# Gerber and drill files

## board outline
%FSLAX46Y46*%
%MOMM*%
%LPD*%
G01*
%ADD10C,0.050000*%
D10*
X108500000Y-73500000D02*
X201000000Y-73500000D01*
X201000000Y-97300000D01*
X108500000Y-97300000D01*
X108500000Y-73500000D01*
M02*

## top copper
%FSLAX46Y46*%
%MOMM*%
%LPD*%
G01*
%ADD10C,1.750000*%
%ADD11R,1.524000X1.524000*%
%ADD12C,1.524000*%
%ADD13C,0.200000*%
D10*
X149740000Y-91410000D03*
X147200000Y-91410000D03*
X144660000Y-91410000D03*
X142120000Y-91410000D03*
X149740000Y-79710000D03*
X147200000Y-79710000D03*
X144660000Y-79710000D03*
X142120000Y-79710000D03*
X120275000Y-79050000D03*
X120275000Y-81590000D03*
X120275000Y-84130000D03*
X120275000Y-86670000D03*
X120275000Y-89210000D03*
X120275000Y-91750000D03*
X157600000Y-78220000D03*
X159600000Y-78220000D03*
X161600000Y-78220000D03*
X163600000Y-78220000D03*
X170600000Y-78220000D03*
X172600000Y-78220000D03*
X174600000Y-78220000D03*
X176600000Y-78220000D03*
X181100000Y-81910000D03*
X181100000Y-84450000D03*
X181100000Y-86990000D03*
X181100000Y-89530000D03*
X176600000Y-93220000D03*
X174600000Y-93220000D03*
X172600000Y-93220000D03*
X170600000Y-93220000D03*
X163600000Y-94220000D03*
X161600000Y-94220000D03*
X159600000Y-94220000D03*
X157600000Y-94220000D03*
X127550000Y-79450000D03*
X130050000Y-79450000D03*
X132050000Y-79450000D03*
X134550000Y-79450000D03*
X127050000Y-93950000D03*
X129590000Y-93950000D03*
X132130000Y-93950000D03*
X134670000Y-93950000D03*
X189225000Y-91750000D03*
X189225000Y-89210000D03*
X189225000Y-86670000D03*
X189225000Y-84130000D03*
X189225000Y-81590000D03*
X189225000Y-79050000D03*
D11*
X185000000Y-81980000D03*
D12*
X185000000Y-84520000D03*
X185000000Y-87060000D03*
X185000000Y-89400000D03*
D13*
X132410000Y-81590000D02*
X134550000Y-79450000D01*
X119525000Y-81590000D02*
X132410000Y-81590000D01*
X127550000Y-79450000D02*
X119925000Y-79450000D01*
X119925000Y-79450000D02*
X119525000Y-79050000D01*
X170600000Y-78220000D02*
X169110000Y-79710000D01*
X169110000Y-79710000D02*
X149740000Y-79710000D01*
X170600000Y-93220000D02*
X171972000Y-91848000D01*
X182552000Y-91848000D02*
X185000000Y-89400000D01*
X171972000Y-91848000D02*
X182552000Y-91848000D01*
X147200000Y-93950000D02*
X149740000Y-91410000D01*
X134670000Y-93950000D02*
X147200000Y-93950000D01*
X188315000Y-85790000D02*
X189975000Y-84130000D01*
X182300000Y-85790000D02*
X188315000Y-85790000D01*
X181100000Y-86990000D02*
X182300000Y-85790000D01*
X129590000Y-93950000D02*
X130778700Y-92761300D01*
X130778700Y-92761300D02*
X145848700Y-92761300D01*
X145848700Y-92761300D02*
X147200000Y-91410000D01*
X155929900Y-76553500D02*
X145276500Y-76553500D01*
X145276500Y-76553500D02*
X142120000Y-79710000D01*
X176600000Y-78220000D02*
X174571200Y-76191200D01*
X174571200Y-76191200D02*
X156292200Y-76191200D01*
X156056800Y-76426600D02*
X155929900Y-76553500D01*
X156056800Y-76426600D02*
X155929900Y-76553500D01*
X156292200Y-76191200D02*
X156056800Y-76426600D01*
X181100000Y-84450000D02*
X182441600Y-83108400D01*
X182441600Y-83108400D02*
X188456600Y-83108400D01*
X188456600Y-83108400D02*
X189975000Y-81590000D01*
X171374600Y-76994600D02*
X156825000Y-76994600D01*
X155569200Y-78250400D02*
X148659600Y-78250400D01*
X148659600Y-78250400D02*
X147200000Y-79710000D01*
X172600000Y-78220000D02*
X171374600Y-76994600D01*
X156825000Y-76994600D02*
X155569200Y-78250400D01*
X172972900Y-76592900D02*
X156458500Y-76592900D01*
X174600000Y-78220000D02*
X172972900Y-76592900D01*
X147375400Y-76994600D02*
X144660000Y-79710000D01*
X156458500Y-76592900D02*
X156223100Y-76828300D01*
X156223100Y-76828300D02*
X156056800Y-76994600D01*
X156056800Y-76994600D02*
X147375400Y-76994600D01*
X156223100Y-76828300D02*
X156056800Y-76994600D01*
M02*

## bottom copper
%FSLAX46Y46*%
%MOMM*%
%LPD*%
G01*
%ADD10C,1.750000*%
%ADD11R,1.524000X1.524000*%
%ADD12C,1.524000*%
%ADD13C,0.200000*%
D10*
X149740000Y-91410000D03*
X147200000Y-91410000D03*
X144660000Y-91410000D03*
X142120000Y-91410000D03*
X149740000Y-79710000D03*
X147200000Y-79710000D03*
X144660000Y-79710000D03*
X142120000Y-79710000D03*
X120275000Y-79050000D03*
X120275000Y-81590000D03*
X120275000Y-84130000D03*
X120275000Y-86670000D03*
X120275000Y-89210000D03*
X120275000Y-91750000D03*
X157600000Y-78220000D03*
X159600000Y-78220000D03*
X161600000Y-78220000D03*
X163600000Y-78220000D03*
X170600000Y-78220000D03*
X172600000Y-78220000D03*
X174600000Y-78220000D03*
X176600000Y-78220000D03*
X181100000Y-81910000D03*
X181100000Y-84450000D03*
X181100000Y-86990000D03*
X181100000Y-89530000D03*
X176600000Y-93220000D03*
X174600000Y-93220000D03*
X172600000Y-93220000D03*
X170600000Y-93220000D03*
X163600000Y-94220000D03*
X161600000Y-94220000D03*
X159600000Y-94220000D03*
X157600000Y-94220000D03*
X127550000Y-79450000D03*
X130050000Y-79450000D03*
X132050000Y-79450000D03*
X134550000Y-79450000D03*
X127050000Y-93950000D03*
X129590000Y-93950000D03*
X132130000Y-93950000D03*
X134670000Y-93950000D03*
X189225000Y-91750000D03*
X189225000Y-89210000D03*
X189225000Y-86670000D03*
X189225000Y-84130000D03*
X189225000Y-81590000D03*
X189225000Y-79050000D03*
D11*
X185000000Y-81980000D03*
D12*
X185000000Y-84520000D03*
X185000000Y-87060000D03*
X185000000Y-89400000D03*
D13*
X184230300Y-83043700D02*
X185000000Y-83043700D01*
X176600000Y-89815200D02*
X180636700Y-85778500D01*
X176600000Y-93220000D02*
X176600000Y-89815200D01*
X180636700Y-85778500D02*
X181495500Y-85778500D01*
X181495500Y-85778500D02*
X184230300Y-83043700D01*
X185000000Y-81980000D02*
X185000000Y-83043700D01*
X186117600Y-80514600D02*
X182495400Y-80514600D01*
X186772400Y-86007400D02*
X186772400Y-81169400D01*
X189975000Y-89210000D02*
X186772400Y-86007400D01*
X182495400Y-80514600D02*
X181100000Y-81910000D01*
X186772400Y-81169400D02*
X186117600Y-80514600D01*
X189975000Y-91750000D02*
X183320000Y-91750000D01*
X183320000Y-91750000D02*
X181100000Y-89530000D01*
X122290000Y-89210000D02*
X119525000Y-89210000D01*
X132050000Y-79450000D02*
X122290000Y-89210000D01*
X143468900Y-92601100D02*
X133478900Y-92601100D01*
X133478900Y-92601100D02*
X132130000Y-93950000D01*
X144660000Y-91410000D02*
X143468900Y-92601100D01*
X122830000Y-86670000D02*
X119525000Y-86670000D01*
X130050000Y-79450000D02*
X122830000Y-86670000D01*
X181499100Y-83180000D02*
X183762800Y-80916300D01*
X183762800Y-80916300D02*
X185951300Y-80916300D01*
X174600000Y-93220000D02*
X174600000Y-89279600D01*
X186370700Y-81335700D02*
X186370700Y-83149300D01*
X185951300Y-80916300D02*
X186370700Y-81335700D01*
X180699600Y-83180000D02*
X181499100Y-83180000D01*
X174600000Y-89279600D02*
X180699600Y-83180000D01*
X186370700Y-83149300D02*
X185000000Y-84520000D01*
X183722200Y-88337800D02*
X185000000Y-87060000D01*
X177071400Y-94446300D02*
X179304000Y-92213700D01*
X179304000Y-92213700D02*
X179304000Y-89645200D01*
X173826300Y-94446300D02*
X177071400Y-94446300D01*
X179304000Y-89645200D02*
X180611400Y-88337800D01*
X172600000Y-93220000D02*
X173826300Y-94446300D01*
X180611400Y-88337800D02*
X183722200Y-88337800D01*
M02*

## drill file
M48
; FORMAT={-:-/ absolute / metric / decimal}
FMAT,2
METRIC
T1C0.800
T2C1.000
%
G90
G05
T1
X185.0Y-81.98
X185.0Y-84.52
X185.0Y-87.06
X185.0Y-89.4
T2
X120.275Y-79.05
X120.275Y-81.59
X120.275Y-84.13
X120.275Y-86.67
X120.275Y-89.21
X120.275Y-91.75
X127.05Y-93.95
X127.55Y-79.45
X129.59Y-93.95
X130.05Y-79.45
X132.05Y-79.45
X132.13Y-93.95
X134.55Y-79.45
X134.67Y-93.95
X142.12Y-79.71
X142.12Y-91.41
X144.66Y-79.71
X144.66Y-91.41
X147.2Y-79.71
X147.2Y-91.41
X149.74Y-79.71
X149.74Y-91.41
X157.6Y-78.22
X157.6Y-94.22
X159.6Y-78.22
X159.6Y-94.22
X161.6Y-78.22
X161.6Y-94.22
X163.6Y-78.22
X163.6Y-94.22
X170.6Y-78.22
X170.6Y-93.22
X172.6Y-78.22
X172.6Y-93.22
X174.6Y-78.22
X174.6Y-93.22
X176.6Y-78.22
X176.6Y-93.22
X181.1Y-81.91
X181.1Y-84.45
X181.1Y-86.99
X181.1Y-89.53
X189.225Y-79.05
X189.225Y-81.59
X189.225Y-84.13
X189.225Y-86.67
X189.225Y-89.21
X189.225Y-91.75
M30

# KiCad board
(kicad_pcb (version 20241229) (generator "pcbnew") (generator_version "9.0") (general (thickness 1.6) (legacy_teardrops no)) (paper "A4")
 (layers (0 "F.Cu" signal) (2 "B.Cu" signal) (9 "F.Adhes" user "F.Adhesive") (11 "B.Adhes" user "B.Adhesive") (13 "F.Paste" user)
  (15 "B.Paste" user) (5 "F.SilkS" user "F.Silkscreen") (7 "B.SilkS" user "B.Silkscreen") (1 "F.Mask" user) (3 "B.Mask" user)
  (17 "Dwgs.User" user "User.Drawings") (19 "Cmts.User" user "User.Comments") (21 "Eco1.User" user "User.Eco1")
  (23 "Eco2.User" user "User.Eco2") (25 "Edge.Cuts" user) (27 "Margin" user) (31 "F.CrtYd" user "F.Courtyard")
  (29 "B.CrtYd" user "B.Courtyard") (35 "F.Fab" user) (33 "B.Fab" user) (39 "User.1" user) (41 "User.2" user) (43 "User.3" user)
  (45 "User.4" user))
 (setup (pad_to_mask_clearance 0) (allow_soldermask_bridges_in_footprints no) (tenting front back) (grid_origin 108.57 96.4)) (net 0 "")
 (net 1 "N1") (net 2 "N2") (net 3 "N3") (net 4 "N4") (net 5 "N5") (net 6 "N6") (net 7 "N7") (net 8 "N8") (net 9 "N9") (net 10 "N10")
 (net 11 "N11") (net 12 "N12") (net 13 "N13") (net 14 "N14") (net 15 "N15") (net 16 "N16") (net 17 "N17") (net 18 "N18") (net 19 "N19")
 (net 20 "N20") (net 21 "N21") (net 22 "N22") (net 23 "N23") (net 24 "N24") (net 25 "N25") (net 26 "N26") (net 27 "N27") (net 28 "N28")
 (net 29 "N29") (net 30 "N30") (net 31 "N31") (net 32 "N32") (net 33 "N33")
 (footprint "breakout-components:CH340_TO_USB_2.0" (layer "F.Cu") (at 151.68 92.91 180)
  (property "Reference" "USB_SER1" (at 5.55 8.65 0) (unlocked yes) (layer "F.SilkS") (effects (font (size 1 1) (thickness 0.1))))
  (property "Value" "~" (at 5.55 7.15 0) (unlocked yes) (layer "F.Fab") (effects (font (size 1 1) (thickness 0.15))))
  (pad "1" thru_hole circle (at 1.94 1.5 180) (size 1.75 1.75) (drill 1) (layers "*.Cu" "*.Mask") (remove_unused_layers no) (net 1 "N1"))
  (pad "2" thru_hole circle (at 4.48 1.5 180) (size 1.75 1.75) (drill 1) (layers "*.Cu" "*.Mask") (remove_unused_layers no) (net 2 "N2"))
  (pad "3" thru_hole circle (at 7.02 1.5 180) (size 1.75 1.75) (drill 1) (layers "*.Cu" "*.Mask") (remove_unused_layers no) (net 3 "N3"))
  (pad "4" thru_hole circle (at 9.56 1.5 180) (size 1.75 1.75) (drill 1) (layers "*.Cu" "*.Mask") (remove_unused_layers no) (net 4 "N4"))
  (pad "5" thru_hole circle (at 1.94 13.2 180) (size 1.75 1.75) (drill 1) (layers "*.Cu" "*.Mask") (remove_unused_layers no) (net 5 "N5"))
  (pad "6" thru_hole circle (at 4.48 13.2 180) (size 1.75 1.75) (drill 1) (layers "*.Cu" "*.Mask") (remove_unused_layers no) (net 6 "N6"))
  (pad "7" thru_hole circle (at 7.02 13.2 180) (size 1.75 1.75) (drill 1) (layers "*.Cu" "*.Mask") (remove_unused_layers no) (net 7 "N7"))
  (pad "8" thru_hole circle (at 9.56 13.2 180) (size 1.75 1.75) (drill 1) (layers "*.Cu" "*.Mask") (remove_unused_layers no) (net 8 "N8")))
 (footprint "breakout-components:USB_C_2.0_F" (layer "F.Cu") (at 108.525 74.5)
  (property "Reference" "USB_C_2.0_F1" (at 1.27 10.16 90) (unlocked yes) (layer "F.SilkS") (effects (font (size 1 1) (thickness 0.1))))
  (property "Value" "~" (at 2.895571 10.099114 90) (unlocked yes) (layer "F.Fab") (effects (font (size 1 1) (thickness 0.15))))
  (pad "1" thru_hole circle (at 11.75 4.55) (size 1.75 1.75) (drill 1) (layers "*.Cu" "*.Mask") (remove_unused_layers no) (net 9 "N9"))
  (pad "2" thru_hole circle (at 11.75 7.09) (size 1.75 1.75) (drill 1) (layers "*.Cu" "*.Mask") (remove_unused_layers no) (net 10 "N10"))
  (pad "3" thru_hole circle (at 11.75 9.63) (size 1.75 1.75) (drill 1) (layers "*.Cu" "*.Mask") (remove_unused_layers no) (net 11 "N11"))
  (pad "4" thru_hole circle (at 11.75 12.17) (size 1.75 1.75) (drill 1) (layers "*.Cu" "*.Mask") (remove_unused_layers no) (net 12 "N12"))
  (pad "5" thru_hole circle (at 11.75 14.71) (size 1.75 1.75) (drill 1) (layers "*.Cu" "*.Mask") (remove_unused_layers no) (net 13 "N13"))
  (pad "6" thru_hole circle (at 11.75 17.25) (size 1.75 1.75) (drill 1) (layers "*.Cu" "*.Mask") (remove_unused_layers no) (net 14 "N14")))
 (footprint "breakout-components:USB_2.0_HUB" (layer "F.Cu") (at 153.6 95.22 90)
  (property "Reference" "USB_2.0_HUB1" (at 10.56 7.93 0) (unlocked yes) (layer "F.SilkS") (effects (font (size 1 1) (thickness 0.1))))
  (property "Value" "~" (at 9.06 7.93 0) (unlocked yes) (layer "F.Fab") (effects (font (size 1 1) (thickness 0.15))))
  (pad "1" thru_hole circle (at 17 4 90) (size 1.75 1.75) (drill 1) (layers "*.Cu" "*.Mask") (remove_unused_layers no) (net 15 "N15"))
  (pad "2" thru_hole circle (at 17 6 90) (size 1.75 1.75) (drill 1) (layers "*.Cu" "*.Mask") (remove_unused_layers no) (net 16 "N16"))
  (pad "3" thru_hole circle (at 17 8 90) (size 1.75 1.75) (drill 1) (layers "*.Cu" "*.Mask") (remove_unused_layers no) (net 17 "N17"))
  (pad "4" thru_hole circle (at 17 10 90) (size 1.75 1.75) (drill 1) (layers "*.Cu" "*.Mask") (remove_unused_layers no) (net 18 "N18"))
  (pad "5" thru_hole circle (at 17 17 90) (size 1.75 1.75) (drill 1) (layers "*.Cu" "*.Mask") (remove_unused_layers no) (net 5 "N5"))
  (pad "6" thru_hole circle (at 17 19 90) (size 1.75 1.75) (drill 1) (layers "*.Cu" "*.Mask") (remove_unused_layers no) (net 6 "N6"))
  (pad "7" thru_hole circle (at 17 21 90) (size 1.75 1.75) (drill 1) (layers "*.Cu" "*.Mask") (remove_unused_layers no) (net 7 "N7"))
  (pad "8" thru_hole circle (at 17 23 90) (size 1.75 1.75) (drill 1) (layers "*.Cu" "*.Mask") (remove_unused_layers no) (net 8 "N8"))
  (pad "9" thru_hole circle (at 13.31 27.5 90) (size 1.75 1.75) (drill 1) (layers "*.Cu" "*.Mask") (remove_unused_layers no) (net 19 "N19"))
  (pad "10" thru_hole circle (at 10.77 27.5 90) (size 1.75 1.75) (drill 1) (layers "*.Cu" "*.Mask") (remove_unused_layers no) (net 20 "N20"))
  (pad "11" thru_hole circle (at 8.23 27.5 90) (size 1.75 1.75) (drill 1) (layers "*.Cu" "*.Mask") (remove_unused_layers no) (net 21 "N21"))
  (pad "12" thru_hole circle (at 5.69 27.5 90) (size 1.75 1.75) (drill 1) (layers "*.Cu" "*.Mask") (remove_unused_layers no) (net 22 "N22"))
  (pad "13" thru_hole circle (at 2 23 90) (size 1.75 1.75) (drill 1) (layers "*.Cu" "*.Mask") (remove_unused_layers no) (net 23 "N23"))
  (pad "14" thru_hole circle (at 2 21 90) (size 1.75 1.75) (drill 1) (layers "*.Cu" "*.Mask") (remove_unused_layers no) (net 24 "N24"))
  (pad "15" thru_hole circle (at 2 19 90) (size 1.75 1.75) (drill 1) (layers "*.Cu" "*.Mask") (remove_unused_layers no) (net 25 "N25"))
  (pad "16" thru_hole circle (at 2 17 90) (size 1.75 1.75) (drill 1) (layers "*.Cu" "*.Mask") (remove_unused_layers no) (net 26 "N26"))
  (pad "17" thru_hole circle (at 1 10 90) (size 1.75 1.75) (drill 1) (layers "*.Cu" "*.Mask") (remove_unused_layers no) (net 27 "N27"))
  (pad "18" thru_hole circle (at 1 8 90) (size 1.75 1.75) (drill 1) (layers "*.Cu" "*.Mask") (remove_unused_layers no) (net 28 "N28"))
  (pad "19" thru_hole circle (at 1 6 90) (size 1.75 1.75) (drill 1) (layers "*.Cu" "*.Mask") (remove_unused_layers no) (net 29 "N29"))
  (pad "20" thru_hole circle (at 1 4 90) (size 1.75 1.75) (drill 1) (layers "*.Cu" "*.Mask") (remove_unused_layers no) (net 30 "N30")))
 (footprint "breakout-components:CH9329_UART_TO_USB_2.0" (layer "F.Cu") (at 123.55 75.45)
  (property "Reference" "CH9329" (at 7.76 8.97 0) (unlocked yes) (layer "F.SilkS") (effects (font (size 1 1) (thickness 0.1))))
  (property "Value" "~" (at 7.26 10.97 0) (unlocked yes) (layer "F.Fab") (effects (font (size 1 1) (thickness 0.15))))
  (pad "1" thru_hole circle (at 4 4) (size 1.75 1.75) (drill 1) (layers "*.Cu" "*.Mask") (remove_unused_layers no) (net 9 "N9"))
  (pad "2" thru_hole circle (at 6.5 4) (size 1.75 1.75) (drill 1) (layers "*.Cu" "*.Mask") (remove_unused_layers no) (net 12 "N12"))
  (pad "3" thru_hole circle (at 8.5 4) (size 1.75 1.75) (drill 1) (layers "*.Cu" "*.Mask") (remove_unused_layers no) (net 13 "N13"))
  (pad "4" thru_hole circle (at 11 4) (size 1.75 1.75) (drill 1) (layers "*.Cu" "*.Mask") (remove_unused_layers no) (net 10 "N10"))
  (pad "5" thru_hole circle (at 3.5 18.5) (size 1.75 1.75) (drill 1) (layers "*.Cu" "*.Mask") (remove_unused_layers no) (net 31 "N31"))
  (pad "6" thru_hole circle (at 6.04 18.5) (size 1.75 1.75) (drill 1) (layers "*.Cu" "*.Mask") (remove_unused_layers no) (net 2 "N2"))
  (pad "7" thru_hole circle (at 8.58 18.5) (size 1.75 1.75) (drill 1) (layers "*.Cu" "*.Mask") (remove_unused_layers no) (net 3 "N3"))
  (pad "8" thru_hole circle (at 11.12 18.5) (size 1.75 1.75) (drill 1) (layers "*.Cu" "*.Mask") (remove_unused_layers no) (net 1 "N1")))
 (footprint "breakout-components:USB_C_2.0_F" (layer "F.Cu") (at 200.975 96.3 180)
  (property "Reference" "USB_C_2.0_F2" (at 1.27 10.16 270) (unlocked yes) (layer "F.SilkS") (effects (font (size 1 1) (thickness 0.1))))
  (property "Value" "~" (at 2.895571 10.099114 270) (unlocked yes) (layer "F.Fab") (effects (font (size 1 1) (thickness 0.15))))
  (pad "1" thru_hole circle (at 11.75 4.55 180) (size 1.75 1.75) (drill 1) (layers "*.Cu" "*.Mask") (remove_unused_layers no) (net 22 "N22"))
  (pad "2" thru_hole circle (at 11.75 7.09 180) (size 1.75 1.75) (drill 1) (layers "*.Cu" "*.Mask") (remove_unused_layers no) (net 19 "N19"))
  (pad "3" thru_hole circle (at 11.75 9.63 180) (size 1.75 1.75) (drill 1) (layers "*.Cu" "*.Mask") (remove_unused_layers no) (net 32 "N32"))
  (pad "4" thru_hole circle (at 11.75 12.17 180) (size 1.75 1.75) (drill 1) (layers "*.Cu" "*.Mask") (remove_unused_layers no)
   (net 21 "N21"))
  (pad "5" thru_hole circle (at 11.75 14.71 180) (size 1.75 1.75) (drill 1) (layers "*.Cu" "*.Mask") (remove_unused_layers no)
   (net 20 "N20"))
  (pad "6" thru_hole circle (at 11.75 17.25 180) (size 1.75 1.75) (drill 1) (layers "*.Cu" "*.Mask") (remove_unused_layers no)
   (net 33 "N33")))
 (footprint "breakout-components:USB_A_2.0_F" (layer "B.Cu") (at 170.8 76.9 -90)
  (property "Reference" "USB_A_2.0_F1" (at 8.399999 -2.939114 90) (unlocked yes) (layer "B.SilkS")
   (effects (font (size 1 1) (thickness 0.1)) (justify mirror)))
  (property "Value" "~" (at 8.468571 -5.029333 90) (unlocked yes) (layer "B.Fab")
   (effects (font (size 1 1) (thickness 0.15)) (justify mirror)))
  (pad "1" thru_hole rect (at 5.08 -14.2 270) (size 1.524 1.524) (drill 0.8) (layers "*.Cu" "*.Mask") (remove_unused_layers no)
   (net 23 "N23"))
  (pad "2" thru_hole circle (at 7.62 -14.2 270) (size 1.524 1.524) (drill 0.8) (layers "*.Cu" "*.Mask") (remove_unused_layers no)
   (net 24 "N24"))
  (pad "3" thru_hole circle (at 10.16 -14.2 270) (size 1.524 1.524) (drill 0.8) (layers "*.Cu" "*.Mask") (remove_unused_layers no)
   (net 25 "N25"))
  (pad "4" thru_hole circle (at 12.5 -14.2 270) (size 1.524 1.524) (drill 0.8) (layers "*.Cu" "*.Mask") (remove_unused_layers no)
   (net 26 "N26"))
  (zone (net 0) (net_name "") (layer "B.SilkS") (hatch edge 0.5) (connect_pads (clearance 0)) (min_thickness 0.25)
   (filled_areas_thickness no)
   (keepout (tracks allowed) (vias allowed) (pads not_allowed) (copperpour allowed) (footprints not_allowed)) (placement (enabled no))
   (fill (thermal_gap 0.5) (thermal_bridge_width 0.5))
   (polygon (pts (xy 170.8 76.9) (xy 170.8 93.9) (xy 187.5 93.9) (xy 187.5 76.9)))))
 (gr_rect (start 108.5 73.5) (end 201 97.3) (stroke (width 0.05) (type default)) (fill no) (layer "Edge.Cuts"))
 (segment (start 132.41 81.59) (end 134.55 79.45) (width 0.2) (layer "F.Cu") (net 10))
 (segment (start 119.525 81.59) (end 132.41 81.59) (width 0.2) (layer "F.Cu") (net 10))
 (segment (start 127.55 79.45) (end 119.925 79.45) (width 0.2) (layer "F.Cu") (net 9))
 (segment (start 119.925 79.45) (end 119.525 79.05) (width 0.2) (layer "F.Cu") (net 9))
 (segment (start 170.6 78.22) (end 169.11 79.71) (width 0.2) (layer "F.Cu") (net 5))
 (segment (start 169.11 79.71) (end 149.74 79.71) (width 0.2) (layer "F.Cu") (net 5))
 (segment (start 184.2303 83.0437) (end 185 83.0437) (width 0.2) (layer "B.Cu") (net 23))
 (segment (start 176.6 89.8152) (end 180.6367 85.7785) (width 0.2) (layer "B.Cu") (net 23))
 (segment (start 176.6 93.22) (end 176.6 89.8152) (width 0.2) (layer "B.Cu") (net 23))
 (segment (start 180.6367 85.7785) (end 181.4955 85.7785) (width 0.2) (layer "B.Cu") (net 23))
 (segment (start 181.4955 85.7785) (end 184.2303 83.0437) (width 0.2) (layer "B.Cu") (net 23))
 (segment (start 185 81.98) (end 185 83.0437) (width 0.2) (layer "B.Cu") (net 23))
 (segment (start 186.1176 80.5146) (end 182.4954 80.5146) (width 0.2) (layer "B.Cu") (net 19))
 (segment (start 186.7724 86.0074) (end 186.7724 81.1694) (width 0.2) (layer "B.Cu") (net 19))
 (segment (start 189.975 89.21) (end 186.7724 86.0074) (width 0.2) (layer "B.Cu") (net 19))
 (segment (start 182.4954 80.5146) (end 181.1 81.91) (width 0.2) (layer "B.Cu") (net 19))
 (segment (start 186.7724 81.1694) (end 186.1176 80.5146) (width 0.2) (layer "B.Cu") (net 19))
 (segment (start 189.975 91.75) (end 183.32 91.75) (width 0.2) (layer "B.Cu") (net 22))
 (segment (start 183.32 91.75) (end 181.1 89.53) (width 0.2) (layer "B.Cu") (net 22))
 (segment (start 170.6 93.22) (end 171.972 91.848) (width 0.2) (layer "F.Cu") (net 26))
 (segment (start 182.552 91.848) (end 185 89.4) (width 0.2) (layer "F.Cu") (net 26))
 (segment (start 171.972 91.848) (end 182.552 91.848) (width 0.2) (layer "F.Cu") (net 26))
 (segment (start 147.2 93.95) (end 149.74 91.41) (width 0.2) (layer "F.Cu") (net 1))
 (segment (start 134.67 93.95) (end 147.2 93.95) (width 0.2) (layer "F.Cu") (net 1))
 (segment (start 122.29 89.21) (end 119.525 89.21) (width 0.2) (layer "B.Cu") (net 13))
 (segment (start 132.05 79.45) (end 122.29 89.21) (width 0.2) (layer "B.Cu") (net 13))
 (segment (start 143.4689 92.6011) (end 133.4789 92.6011) (width 0.2) (layer "B.Cu") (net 3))
 (segment (start 133.4789 92.6011) (end 132.13 93.95) (width 0.2) (layer "B.Cu") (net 3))
 (segment (start 144.66 91.41) (end 143.4689 92.6011) (width 0.2) (layer "B.Cu") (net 3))
 (segment (start 188.315 85.79) (end 189.975 84.13) (width 0.2) (layer "F.Cu") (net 21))
 (segment (start 182.3 85.79) (end 188.315 85.79) (width 0.2) (layer "F.Cu") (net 21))
 (segment (start 181.1 86.99) (end 182.3 85.79) (width 0.2) (layer "F.Cu") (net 21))
 (segment (start 129.59 93.95) (end 130.7787 92.7613) (width 0.2) (layer "F.Cu") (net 2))
 (segment (start 130.7787 92.7613) (end 145.8487 92.7613) (width 0.2) (layer "F.Cu") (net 2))
 (segment (start 145.8487 92.7613) (end 147.2 91.41) (width 0.2) (layer "F.Cu") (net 2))
 (segment (start 122.83 86.67) (end 119.525 86.67) (width 0.2) (layer "B.Cu") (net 12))
 (segment (start 130.05 79.45) (end 122.83 86.67) (width 0.2) (layer "B.Cu") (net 12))
 (segment (start 181.4991 83.18) (end 183.7628 80.9163) (width 0.2) (layer "B.Cu") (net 24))
 (segment (start 183.7628 80.9163) (end 185.9513 80.9163) (width 0.2) (layer "B.Cu") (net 24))
 (segment (start 174.6 93.22) (end 174.6 89.2796) (width 0.2) (layer "B.Cu") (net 24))
 (segment (start 186.3707 81.3357) (end 186.3707 83.1493) (width 0.2) (layer "B.Cu") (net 24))
 (segment (start 185.9513 80.9163) (end 186.3707 81.3357) (width 0.2) (layer "B.Cu") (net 24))
 (segment (start 180.6996 83.18) (end 181.4991 83.18) (width 0.2) (layer "B.Cu") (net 24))
 (segment (start 174.6 89.2796) (end 180.6996 83.18) (width 0.2) (layer "B.Cu") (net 24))
 (segment (start 186.3707 83.1493) (end 185 84.52) (width 0.2) (layer "B.Cu") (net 24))
 (segment (start 155.9299 76.5535) (end 145.2765 76.5535) (width 0.2) (layer "F.Cu") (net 8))
 (segment (start 145.2765 76.5535) (end 142.12 79.71) (width 0.2) (layer "F.Cu") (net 8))
 (segment (start 176.6 78.22) (end 174.5712 76.1912) (width 0.2) (layer "F.Cu") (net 8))
 (segment (start 174.5712 76.1912) (end 156.2922 76.1912) (width 0.2) (layer "F.Cu") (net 8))
 (segment (start 156.0568 76.4266) (end 155.9299 76.5535) (width 0.2) (layer "F.Cu") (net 8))
 (segment (start 156.0568 76.4266) (end 155.9299 76.5535) (width 0.2) (layer "F.Cu") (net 8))
 (segment (start 156.2922 76.1912) (end 156.0568 76.4266) (width 0.2) (layer "F.Cu") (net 8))
 (segment (start 181.1 84.45) (end 182.4416 83.1084) (width 0.2) (layer "F.Cu") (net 20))
 (segment (start 182.4416 83.1084) (end 188.4566 83.1084) (width 0.2) (layer "F.Cu") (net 20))
 (segment (start 188.4566 83.1084) (end 189.975 81.59) (width 0.2) (layer "F.Cu") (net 20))
 (segment (start 171.3746 76.9946) (end 156.825 76.9946) (width 0.2) (layer "F.Cu") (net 6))
 (segment (start 155.5692 78.2504) (end 148.6596 78.2504) (width 0.2) (layer "F.Cu") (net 6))
 (segment (start 148.6596 78.2504) (end 147.2 79.71) (width 0.2) (layer "F.Cu") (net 6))
 (segment (start 172.6 78.22) (end 171.3746 76.9946) (width 0.2) (layer "F.Cu") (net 6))
 (segment (start 156.825 76.9946) (end 155.5692 78.2504) (width 0.2) (layer "F.Cu") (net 6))
 (segment (start 172.9729 76.5929) (end 156.4585 76.5929) (width 0.2) (layer "F.Cu") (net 7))
 (segment (start 174.6 78.22) (end 172.9729 76.5929) (width 0.2) (layer "F.Cu") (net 7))
 (segment (start 147.3754 76.9946) (end 144.66 79.71) (width 0.2) (layer "F.Cu") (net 7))
 (segment (start 156.4585 76.5929) (end 156.2231 76.8283) (width 0.2) (layer "F.Cu") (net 7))
 (segment (start 156.2231 76.8283) (end 156.0568 76.9946) (width 0.2) (layer "F.Cu") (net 7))
 (segment (start 156.0568 76.9946) (end 147.3754 76.9946) (width 0.2) (layer "F.Cu") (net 7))
 (segment (start 156.2231 76.8283) (end 156.0568 76.9946) (width 0.2) (layer "F.Cu") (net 7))
 (segment (start 183.7222 88.3378) (end 185 87.06) (width 0.2) (layer "B.Cu") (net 25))
 (segment (start 177.0714 94.4463) (end 179.304 92.2137) (width 0.2) (layer "B.Cu") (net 25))
 (segment (start 179.304 92.2137) (end 179.304 89.6452) (width 0.2) (layer "B.Cu") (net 25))
 (segment (start 173.8263 94.4463) (end 177.0714 94.4463) (width 0.2) (layer "B.Cu") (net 25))
 (segment (start 179.304 89.6452) (end 180.6114 88.3378) (width 0.2) (layer "B.Cu") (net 25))
 (segment (start 172.6 93.22) (end 173.8263 94.4463) (width 0.2) (layer "B.Cu") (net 25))
 (segment (start 180.6114 88.3378) (end 183.7222 88.3378) (width 0.2) (layer "B.Cu") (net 25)))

